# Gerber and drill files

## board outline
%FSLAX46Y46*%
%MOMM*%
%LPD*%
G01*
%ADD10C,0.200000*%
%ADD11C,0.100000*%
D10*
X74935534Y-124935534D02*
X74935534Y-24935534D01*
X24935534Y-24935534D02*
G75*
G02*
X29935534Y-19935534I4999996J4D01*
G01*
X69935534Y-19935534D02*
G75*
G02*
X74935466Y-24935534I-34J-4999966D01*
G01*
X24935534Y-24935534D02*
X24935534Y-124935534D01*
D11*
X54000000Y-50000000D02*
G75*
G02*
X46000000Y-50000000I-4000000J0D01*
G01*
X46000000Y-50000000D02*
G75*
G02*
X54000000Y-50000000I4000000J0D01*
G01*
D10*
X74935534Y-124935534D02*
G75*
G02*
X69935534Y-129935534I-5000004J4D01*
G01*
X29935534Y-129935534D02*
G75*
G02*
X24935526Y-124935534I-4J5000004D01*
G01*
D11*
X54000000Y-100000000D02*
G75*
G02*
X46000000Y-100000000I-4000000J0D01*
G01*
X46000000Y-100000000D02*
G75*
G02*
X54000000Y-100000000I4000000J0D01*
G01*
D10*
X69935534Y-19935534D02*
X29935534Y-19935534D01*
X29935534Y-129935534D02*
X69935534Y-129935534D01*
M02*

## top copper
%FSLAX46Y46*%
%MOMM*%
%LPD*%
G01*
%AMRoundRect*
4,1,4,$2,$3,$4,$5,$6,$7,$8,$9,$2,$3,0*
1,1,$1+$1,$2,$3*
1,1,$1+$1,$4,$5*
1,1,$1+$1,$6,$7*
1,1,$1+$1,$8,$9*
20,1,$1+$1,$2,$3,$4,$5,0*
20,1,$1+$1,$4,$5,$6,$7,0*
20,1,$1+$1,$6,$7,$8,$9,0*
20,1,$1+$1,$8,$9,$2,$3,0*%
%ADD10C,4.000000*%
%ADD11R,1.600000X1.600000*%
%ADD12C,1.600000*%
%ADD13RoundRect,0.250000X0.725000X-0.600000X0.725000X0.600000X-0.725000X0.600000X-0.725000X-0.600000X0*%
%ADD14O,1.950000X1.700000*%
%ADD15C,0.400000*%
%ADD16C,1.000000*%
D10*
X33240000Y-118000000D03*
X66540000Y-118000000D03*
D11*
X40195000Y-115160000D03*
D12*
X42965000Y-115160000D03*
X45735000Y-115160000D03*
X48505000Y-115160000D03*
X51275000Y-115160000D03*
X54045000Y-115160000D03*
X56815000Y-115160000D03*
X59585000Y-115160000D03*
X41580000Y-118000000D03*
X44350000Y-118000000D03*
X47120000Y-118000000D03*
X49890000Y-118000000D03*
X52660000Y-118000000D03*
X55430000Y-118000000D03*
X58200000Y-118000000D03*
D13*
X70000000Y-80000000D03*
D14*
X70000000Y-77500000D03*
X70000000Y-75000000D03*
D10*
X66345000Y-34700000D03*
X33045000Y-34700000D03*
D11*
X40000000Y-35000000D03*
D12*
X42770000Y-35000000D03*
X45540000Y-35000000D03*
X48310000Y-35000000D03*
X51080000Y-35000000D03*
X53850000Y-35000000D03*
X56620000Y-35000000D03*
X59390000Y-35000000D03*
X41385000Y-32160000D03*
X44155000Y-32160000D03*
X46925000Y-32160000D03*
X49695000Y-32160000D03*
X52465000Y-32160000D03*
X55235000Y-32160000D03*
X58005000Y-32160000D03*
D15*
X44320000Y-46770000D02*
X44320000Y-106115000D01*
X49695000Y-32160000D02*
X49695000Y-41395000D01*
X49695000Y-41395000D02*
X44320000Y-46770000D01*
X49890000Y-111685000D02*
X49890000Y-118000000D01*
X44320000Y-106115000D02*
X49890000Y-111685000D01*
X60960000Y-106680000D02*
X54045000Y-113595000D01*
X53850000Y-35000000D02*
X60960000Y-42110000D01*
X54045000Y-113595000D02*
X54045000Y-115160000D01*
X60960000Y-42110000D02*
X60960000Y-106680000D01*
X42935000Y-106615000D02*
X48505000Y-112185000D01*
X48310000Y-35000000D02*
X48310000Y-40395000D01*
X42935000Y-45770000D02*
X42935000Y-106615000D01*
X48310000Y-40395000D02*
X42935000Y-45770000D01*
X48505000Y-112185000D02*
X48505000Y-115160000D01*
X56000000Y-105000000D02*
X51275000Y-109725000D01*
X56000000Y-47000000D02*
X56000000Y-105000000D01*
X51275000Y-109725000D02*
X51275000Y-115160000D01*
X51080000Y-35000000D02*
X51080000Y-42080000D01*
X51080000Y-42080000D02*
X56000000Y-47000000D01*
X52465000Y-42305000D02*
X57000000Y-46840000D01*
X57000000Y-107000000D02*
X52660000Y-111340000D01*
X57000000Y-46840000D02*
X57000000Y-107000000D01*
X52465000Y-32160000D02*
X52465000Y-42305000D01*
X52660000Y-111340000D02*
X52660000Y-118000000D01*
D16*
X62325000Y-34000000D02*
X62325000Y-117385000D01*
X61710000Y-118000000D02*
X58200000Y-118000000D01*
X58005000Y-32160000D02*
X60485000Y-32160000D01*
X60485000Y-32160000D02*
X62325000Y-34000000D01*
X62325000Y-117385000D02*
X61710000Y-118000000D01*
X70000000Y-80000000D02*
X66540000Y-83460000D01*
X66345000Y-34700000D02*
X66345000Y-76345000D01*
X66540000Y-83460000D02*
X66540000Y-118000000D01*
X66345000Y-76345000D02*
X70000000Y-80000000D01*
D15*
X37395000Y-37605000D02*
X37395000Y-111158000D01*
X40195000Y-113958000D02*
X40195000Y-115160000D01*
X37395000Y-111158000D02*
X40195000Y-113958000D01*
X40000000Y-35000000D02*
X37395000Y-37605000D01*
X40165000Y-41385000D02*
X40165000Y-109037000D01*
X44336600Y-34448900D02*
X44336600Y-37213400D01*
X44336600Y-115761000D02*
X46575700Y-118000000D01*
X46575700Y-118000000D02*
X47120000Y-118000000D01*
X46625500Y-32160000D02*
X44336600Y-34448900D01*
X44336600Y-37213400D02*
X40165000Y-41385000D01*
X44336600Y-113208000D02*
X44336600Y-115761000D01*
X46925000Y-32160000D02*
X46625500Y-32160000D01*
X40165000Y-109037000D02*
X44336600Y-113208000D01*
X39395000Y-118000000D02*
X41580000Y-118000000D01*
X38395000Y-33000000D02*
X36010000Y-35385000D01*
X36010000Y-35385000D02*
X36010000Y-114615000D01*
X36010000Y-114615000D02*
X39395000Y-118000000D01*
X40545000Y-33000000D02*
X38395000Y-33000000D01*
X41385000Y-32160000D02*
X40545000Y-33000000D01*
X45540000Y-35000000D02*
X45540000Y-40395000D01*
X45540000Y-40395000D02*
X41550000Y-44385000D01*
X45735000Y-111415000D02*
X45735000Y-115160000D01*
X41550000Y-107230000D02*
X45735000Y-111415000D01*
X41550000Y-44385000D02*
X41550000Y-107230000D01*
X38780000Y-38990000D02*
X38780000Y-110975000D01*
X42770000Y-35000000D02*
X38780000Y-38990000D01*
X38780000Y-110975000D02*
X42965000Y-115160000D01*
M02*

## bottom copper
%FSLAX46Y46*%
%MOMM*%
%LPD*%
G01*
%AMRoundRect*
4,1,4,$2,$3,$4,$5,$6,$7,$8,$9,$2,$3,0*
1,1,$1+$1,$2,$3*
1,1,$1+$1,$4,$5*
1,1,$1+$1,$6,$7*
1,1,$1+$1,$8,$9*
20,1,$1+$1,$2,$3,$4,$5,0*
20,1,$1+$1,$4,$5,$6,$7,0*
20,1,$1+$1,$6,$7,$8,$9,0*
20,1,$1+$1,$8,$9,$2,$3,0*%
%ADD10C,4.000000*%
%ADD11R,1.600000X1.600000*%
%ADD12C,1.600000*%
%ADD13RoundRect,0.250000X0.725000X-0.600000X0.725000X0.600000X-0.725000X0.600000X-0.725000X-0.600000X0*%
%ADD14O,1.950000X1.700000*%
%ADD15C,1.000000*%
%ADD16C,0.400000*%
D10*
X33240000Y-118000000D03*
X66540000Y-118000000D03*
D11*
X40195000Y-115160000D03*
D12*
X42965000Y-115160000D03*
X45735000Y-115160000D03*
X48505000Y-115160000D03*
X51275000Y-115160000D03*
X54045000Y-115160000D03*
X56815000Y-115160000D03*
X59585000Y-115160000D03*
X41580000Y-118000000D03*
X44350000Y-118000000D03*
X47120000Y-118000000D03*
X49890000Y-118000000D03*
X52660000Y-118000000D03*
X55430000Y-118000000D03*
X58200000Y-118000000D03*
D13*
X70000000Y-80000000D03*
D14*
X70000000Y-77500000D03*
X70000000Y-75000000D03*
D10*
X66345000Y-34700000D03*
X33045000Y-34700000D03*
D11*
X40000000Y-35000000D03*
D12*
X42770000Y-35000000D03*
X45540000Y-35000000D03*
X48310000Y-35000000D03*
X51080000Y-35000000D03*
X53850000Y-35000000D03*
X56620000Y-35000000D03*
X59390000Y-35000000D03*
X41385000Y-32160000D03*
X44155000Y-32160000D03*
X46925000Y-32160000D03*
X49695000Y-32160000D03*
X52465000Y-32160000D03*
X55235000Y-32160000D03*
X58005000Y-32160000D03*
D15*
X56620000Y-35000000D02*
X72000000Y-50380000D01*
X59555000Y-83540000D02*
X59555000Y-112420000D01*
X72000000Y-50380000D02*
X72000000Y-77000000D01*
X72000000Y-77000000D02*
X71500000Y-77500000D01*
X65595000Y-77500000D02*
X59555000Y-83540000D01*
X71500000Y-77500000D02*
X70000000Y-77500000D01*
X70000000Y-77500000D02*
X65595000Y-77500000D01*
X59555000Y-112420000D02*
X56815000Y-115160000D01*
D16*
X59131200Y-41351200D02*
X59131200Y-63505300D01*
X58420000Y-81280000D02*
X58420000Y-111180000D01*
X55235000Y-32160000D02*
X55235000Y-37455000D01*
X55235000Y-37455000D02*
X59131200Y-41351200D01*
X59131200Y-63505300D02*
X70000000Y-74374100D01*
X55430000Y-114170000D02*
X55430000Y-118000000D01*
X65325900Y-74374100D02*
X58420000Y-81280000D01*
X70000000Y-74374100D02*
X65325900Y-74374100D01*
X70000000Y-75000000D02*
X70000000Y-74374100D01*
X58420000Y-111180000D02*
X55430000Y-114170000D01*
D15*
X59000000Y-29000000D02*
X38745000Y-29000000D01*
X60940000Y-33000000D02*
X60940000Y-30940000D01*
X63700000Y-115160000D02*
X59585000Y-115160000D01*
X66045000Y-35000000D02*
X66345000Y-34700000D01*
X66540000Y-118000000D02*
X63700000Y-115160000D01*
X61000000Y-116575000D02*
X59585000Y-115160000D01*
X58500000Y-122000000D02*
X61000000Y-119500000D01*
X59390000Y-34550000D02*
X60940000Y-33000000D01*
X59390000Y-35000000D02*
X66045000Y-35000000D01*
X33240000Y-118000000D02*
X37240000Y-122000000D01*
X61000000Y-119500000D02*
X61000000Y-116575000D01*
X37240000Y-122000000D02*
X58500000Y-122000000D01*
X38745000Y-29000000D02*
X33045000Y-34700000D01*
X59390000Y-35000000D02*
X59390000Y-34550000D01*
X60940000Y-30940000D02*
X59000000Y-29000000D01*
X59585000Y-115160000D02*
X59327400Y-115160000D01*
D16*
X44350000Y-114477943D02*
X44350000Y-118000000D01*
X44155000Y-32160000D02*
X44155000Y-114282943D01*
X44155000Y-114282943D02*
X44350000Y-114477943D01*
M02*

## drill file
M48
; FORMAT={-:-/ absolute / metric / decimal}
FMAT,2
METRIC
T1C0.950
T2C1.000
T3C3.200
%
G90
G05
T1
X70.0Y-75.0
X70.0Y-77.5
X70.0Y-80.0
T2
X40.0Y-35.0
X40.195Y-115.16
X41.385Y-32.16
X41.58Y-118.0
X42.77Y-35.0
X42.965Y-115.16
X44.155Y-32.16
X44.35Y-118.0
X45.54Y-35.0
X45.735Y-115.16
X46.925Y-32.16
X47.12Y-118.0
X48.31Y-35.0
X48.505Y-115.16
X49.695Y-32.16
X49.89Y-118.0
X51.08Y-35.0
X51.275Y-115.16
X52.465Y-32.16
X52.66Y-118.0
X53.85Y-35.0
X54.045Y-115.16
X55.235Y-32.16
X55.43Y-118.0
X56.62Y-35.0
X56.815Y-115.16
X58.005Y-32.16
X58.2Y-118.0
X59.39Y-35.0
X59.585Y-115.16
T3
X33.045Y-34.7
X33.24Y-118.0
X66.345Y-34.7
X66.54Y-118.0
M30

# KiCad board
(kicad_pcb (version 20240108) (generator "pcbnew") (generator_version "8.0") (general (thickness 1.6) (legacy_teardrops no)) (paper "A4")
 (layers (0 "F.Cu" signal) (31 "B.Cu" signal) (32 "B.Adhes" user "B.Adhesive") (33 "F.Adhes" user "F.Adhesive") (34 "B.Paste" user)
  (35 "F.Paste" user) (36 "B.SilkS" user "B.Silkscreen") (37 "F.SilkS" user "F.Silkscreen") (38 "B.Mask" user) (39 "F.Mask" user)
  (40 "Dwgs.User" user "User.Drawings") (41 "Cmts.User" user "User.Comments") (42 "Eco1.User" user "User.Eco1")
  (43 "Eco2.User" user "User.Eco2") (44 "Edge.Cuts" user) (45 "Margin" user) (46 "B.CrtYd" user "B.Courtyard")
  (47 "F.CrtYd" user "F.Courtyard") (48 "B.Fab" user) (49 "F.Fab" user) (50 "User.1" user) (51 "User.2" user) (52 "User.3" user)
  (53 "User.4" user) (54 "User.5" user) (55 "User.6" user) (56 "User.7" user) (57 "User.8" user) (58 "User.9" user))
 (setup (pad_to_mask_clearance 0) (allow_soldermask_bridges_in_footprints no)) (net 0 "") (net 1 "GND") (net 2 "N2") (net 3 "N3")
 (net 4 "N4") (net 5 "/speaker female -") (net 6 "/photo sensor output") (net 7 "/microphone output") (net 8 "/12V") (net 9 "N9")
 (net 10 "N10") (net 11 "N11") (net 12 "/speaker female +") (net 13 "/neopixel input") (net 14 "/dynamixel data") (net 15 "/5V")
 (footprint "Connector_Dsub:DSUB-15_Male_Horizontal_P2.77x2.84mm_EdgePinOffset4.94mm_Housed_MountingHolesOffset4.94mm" (layer "F.Cu")
  (at 40.195 115.16)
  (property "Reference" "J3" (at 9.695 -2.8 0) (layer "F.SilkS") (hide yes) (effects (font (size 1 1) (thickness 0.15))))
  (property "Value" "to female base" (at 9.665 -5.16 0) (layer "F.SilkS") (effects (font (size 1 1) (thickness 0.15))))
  (pad "0" thru_hole circle (at -6.955 2.84) (size 4 4) (drill 3.2) (layers "*.Cu" "*.Mask") (remove_unused_layers no) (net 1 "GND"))
  (pad "0" thru_hole circle (at 26.345 2.84) (size 4 4) (drill 3.2) (layers "*.Cu" "*.Mask") (remove_unused_layers no) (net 1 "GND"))
  (pad "1" thru_hole rect (at 0 0) (size 1.6 1.6) (drill 1) (layers "*.Cu" "*.Mask") (remove_unused_layers no) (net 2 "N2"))
  (pad "2" thru_hole circle (at 2.77 0) (size 1.6 1.6) (drill 1) (layers "*.Cu" "*.Mask") (remove_unused_layers no) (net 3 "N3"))
  (pad "3" thru_hole circle (at 5.54 0) (size 1.6 1.6) (drill 1) (layers "*.Cu" "*.Mask") (remove_unused_layers no) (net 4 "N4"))
  (pad "4" thru_hole circle (at 8.31 0) (size 1.6 1.6) (drill 1) (layers "*.Cu" "*.Mask") (remove_unused_layers no)
   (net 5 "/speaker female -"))
  (pad "5" thru_hole circle (at 11.08 0) (size 1.6 1.6) (drill 1) (layers "*.Cu" "*.Mask") (remove_unused_layers no)
   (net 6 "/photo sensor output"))
  (pad "6" thru_hole circle (at 13.85 0) (size 1.6 1.6) (drill 1) (layers "*.Cu" "*.Mask") (remove_unused_layers no)
   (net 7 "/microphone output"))
  (pad "7" thru_hole circle (at 16.62 0) (size 1.6 1.6) (drill 1) (layers "*.Cu" "*.Mask") (remove_unused_layers no) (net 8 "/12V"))
  (pad "8" thru_hole circle (at 19.39 0) (size 1.6 1.6) (drill 1) (layers "*.Cu" "*.Mask") (remove_unused_layers no) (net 1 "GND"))
  (pad "9" thru_hole circle (at 1.385 2.84) (size 1.6 1.6) (drill 1) (layers "*.Cu" "*.Mask") (remove_unused_layers no) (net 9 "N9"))
  (pad "10" thru_hole circle (at 4.155 2.84) (size 1.6 1.6) (drill 1) (layers "*.Cu" "*.Mask") (remove_unused_layers no) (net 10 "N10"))
  (pad "11" thru_hole circle (at 6.925 2.84) (size 1.6 1.6) (drill 1) (layers "*.Cu" "*.Mask") (remove_unused_layers no) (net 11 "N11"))
  (pad "12" thru_hole circle (at 9.695 2.84) (size 1.6 1.6) (drill 1) (layers "*.Cu" "*.Mask") (remove_unused_layers no)
   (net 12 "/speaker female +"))
  (pad "13" thru_hole circle (at 12.465 2.84) (size 1.6 1.6) (drill 1) (layers "*.Cu" "*.Mask") (remove_unused_layers no)
   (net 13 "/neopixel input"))
  (pad "14" thru_hole circle (at 15.235 2.84) (size 1.6 1.6) (drill 1) (layers "*.Cu" "*.Mask") (remove_unused_layers no)
   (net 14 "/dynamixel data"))
  (pad "15" thru_hole circle (at 18.005 2.84) (size 1.6 1.6) (drill 1) (layers "*.Cu" "*.Mask") (remove_unused_layers no) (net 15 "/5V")))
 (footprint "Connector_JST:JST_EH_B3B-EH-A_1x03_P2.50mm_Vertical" (layer "F.Cu") (at 70 80 90)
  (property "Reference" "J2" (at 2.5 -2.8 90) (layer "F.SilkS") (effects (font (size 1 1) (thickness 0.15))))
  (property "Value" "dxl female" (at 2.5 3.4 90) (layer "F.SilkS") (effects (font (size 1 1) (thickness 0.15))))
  (pad "1" thru_hole roundrect (at 0 0 90) (size 1.7 1.95) (drill 0.95) (layers "*.Cu" "*.Mask") (remove_unused_layers no)
   (roundrect_rratio 0.147059) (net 1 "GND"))
  (pad "2" thru_hole oval (at 2.5 0 90) (size 1.7 1.95) (drill 0.95) (layers "*.Cu" "*.Mask") (remove_unused_layers no) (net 8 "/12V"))
  (pad "3" thru_hole oval (at 5 0 90) (size 1.7 1.95) (drill 0.95) (layers "*.Cu" "*.Mask") (remove_unused_layers no)
   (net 14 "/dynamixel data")))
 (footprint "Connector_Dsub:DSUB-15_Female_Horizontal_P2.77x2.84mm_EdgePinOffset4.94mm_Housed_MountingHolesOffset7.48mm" (layer "F.Cu")
  (at 40 35 180)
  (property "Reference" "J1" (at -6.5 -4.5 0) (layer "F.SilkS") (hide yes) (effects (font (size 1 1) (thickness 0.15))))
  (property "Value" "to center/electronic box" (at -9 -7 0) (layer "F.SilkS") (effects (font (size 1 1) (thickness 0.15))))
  (pad "0" thru_hole circle (at -26.345 0.3 180) (size 4 4) (drill 3.2) (layers "*.Cu" "*.Mask") (remove_unused_layers no) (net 1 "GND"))
  (pad "0" thru_hole circle (at 6.955 0.3 180) (size 4 4) (drill 3.2) (layers "*.Cu" "*.Mask") (remove_unused_layers no) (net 1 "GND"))
  (pad "1" thru_hole rect (at 0 0 180) (size 1.6 1.6) (drill 1) (layers "*.Cu" "*.Mask") (remove_unused_layers no) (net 2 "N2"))
  (pad "2" thru_hole circle (at -2.77 0 180) (size 1.6 1.6) (drill 1) (layers "*.Cu" "*.Mask") (remove_unused_layers no) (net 3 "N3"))
  (pad "3" thru_hole circle (at -5.54 0 180) (size 1.6 1.6) (drill 1) (layers "*.Cu" "*.Mask") (remove_unused_layers no) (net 4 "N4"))
  (pad "4" thru_hole circle (at -8.31 0 180) (size 1.6 1.6) (drill 1) (layers "*.Cu" "*.Mask") (remove_unused_layers no)
   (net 5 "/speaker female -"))
  (pad "5" thru_hole circle (at -11.08 0 180) (size 1.6 1.6) (drill 1) (layers "*.Cu" "*.Mask") (remove_unused_layers no)
   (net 6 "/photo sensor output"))
  (pad "6" thru_hole circle (at -13.85 0 180) (size 1.6 1.6) (drill 1) (layers "*.Cu" "*.Mask") (remove_unused_layers no)
   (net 7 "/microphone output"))
  (pad "7" thru_hole circle (at -16.62 0 180) (size 1.6 1.6) (drill 1) (layers "*.Cu" "*.Mask") (remove_unused_layers no) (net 8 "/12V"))
  (pad "8" thru_hole circle (at -19.39 0 180) (size 1.6 1.6) (drill 1) (layers "*.Cu" "*.Mask") (remove_unused_layers no) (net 1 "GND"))
  (pad "9" thru_hole circle (at -1.385 2.84 180) (size 1.6 1.6) (drill 1) (layers "*.Cu" "*.Mask") (remove_unused_layers no) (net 9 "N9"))
  (pad "10" thru_hole circle (at -4.155 2.84 180) (size 1.6 1.6) (drill 1) (layers "*.Cu" "*.Mask") (remove_unused_layers no) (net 10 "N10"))
  (pad "11" thru_hole circle (at -6.925 2.84 180) (size 1.6 1.6) (drill 1) (layers "*.Cu" "*.Mask") (remove_unused_layers no) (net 11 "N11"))
  (pad "12" thru_hole circle (at -9.695 2.84 180) (size 1.6 1.6) (drill 1) (layers "*.Cu" "*.Mask") (remove_unused_layers no)
   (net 12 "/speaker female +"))
  (pad "13" thru_hole circle (at -12.465 2.84 180) (size 1.6 1.6) (drill 1) (layers "*.Cu" "*.Mask") (remove_unused_layers no)
   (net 13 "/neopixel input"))
  (pad "14" thru_hole circle (at -15.235 2.84 180) (size 1.6 1.6) (drill 1) (layers "*.Cu" "*.Mask") (remove_unused_layers no)
   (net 14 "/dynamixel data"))
  (pad "15" thru_hole circle (at -18.005 2.84 180) (size 1.6 1.6) (drill 1) (layers "*.Cu" "*.Mask") (remove_unused_layers no)
   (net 15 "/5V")))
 (gr_line (start 74.935534 124.935534) (end 74.935534 24.935534) (stroke (width 0.2) (type default)) (layer "Edge.Cuts"))
 (gr_arc (start 24.935534 24.935534) (mid 26.4 21.4) (end 29.935534 19.935534) (stroke (width 0.2) (type default)) (layer "Edge.Cuts"))
 (gr_arc (start 69.935534 19.935534) (mid 73.471068 21.4) (end 74.935534 24.935534) (stroke (width 0.2) (type default)) (layer "Edge.Cuts"))
 (gr_line (start 24.935534 24.935534) (end 24.935534 124.935534) (stroke (width 0.2) (type default)) (layer "Edge.Cuts"))
 (gr_circle (center 50 50) (end 54 50) (stroke (width 0.1) (type default)) (fill none) (layer "Edge.Cuts"))
 (gr_arc (start 74.935534 124.935534) (mid 73.471068 128.471068) (end 69.935534 129.935534) (stroke (width 0.2) (type default))
  (layer "Edge.Cuts"))
 (gr_arc (start 29.935534 129.935534) (mid 26.4 128.471068) (end 24.935534 124.935534) (stroke (width 0.2) (type default))
  (layer "Edge.Cuts"))
 (gr_circle (center 50 100) (end 54 100) (stroke (width 0.1) (type default)) (fill none) (layer "Edge.Cuts"))
 (gr_line (start 69.935534 19.935534) (end 29.935534 19.935534) (stroke (width 0.2) (type default)) (layer "Edge.Cuts"))
 (gr_line (start 29.935534 129.935534) (end 69.935534 129.935534) (stroke (width 0.2) (type default)) (layer "Edge.Cuts"))
 (segment (start 44.32 46.77) (end 44.32 106.115) (width 0.4) (layer "F.Cu") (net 12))
 (segment (start 49.695 32.16) (end 49.695 41.395) (width 0.4) (layer "F.Cu") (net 12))
 (segment (start 49.695 41.395) (end 44.32 46.77) (width 0.4) (layer "F.Cu") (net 12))
 (segment (start 49.89 111.685) (end 49.89 118) (width 0.4) (layer "F.Cu") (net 12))
 (segment (start 44.32 106.115) (end 49.89 111.685) (width 0.4) (layer "F.Cu") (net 12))
 (segment (start 56.62 35) (end 72 50.38) (width 1) (layer "B.Cu") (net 8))
 (segment (start 59.555 83.54) (end 59.555 112.42) (width 1) (layer "B.Cu") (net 8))
 (segment (start 72 50.38) (end 72 77) (width 1) (layer "B.Cu") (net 8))
 (segment (start 72 77) (end 71.5 77.5) (width 1) (layer "B.Cu") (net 8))
 (segment (start 65.595 77.5) (end 59.555 83.54) (width 1) (layer "B.Cu") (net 8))
 (segment (start 71.5 77.5) (end 70 77.5) (width 1) (layer "B.Cu") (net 8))
 (segment (start 70 77.5) (end 65.595 77.5) (width 1) (layer "B.Cu") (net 8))
 (segment (start 59.555 112.42) (end 56.815 115.16) (width 1) (layer "B.Cu") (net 8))
 (segment (start 59.1312 41.3512) (end 59.1312 63.5053) (width 0.4) (layer "B.Cu") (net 14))
 (segment (start 58.42 81.28) (end 58.42 111.18) (width 0.4) (layer "B.Cu") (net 14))
 (segment (start 55.235 32.16) (end 55.235 37.455) (width 0.4) (layer "B.Cu") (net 14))
 (segment (start 55.235 37.455) (end 59.1312 41.3512) (width 0.4) (layer "B.Cu") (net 14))
 (segment (start 59.1312 63.5053) (end 70 74.3741) (width 0.4) (layer "B.Cu") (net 14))
 (segment (start 55.43 114.17) (end 55.43 118) (width 0.4) (layer "B.Cu") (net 14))
 (segment (start 65.3259 74.3741) (end 58.42 81.28) (width 0.4) (layer "B.Cu") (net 14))
 (segment (start 70 74.3741) (end 65.3259 74.3741) (width 0.4) (layer "B.Cu") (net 14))
 (segment (start 70 75) (end 70 74.3741) (width 0.4) (layer "B.Cu") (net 14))
 (segment (start 58.42 111.18) (end 55.43 114.17) (width 0.4) (layer "B.Cu") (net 14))
 (segment (start 60.96 106.68) (end 54.045 113.595) (width 0.4) (layer "F.Cu") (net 7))
 (segment (start 53.85 35) (end 60.96 42.11) (width 0.4) (layer "F.Cu") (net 7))
 (segment (start 54.045 113.595) (end 54.045 115.16) (width 0.4) (layer "F.Cu") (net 7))
 (segment (start 60.96 42.11) (end 60.96 106.68) (width 0.4) (layer "F.Cu") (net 7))
 (segment (start 42.935 106.615) (end 48.505 112.185) (width 0.4) (layer "F.Cu") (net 5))
 (segment (start 48.31 35) (end 48.31 40.395) (width 0.4) (layer "F.Cu") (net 5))
 (segment (start 42.935 45.77) (end 42.935 106.615) (width 0.4) (layer "F.Cu") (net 5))
 (segment (start 48.31 40.395) (end 42.935 45.77) (width 0.4) (layer "F.Cu") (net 5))
 (segment (start 48.505 112.185) (end 48.505 115.16) (width 0.4) (layer "F.Cu") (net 5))
 (segment (start 56 105) (end 51.275 109.725) (width 0.4) (layer "F.Cu") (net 6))
 (segment (start 56 47) (end 56 105) (width 0.4) (layer "F.Cu") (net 6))
 (segment (start 51.275 109.725) (end 51.275 115.16) (width 0.4) (layer "F.Cu") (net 6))
 (segment (start 51.08 35) (end 51.08 42.08) (width 0.4) (layer "F.Cu") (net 6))
 (segment (start 51.08 42.08) (end 56 47) (width 0.4) (layer "F.Cu") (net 6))
 (segment (start 52.465 42.305) (end 57 46.84) (width 0.4) (layer "F.Cu") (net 13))
 (segment (start 57 107) (end 52.66 111.34) (width 0.4) (layer "F.Cu") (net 13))
 (segment (start 57 46.84) (end 57 107) (width 0.4) (layer "F.Cu") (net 13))
 (segment (start 52.465 32.16) (end 52.465 42.305) (width 0.4) (layer "F.Cu") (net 13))
 (segment (start 52.66 111.34) (end 52.66 118) (width 0.4) (layer "F.Cu") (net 13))
 (segment (start 62.325 34) (end 62.325 117.385) (width 1) (layer "F.Cu") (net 15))
 (segment (start 61.71 118) (end 58.2 118) (width 1) (layer "F.Cu") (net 15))
 (segment (start 58.005 32.16) (end 60.485 32.16) (width 1) (layer "F.Cu") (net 15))
 (segment (start 60.485 32.16) (end 62.325 34) (width 1) (layer "F.Cu") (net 15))
 (segment (start 62.325 117.385) (end 61.71 118) (width 1) (layer "F.Cu") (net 15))
 (segment (start 70 80) (end 66.54 83.46) (width 1) (layer "F.Cu") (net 1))
 (segment (start 66.345 34.7) (end 66.345 76.345) (width 1) (layer "F.Cu") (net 1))
 (segment (start 66.54 83.46) (end 66.54 118) (width 1) (layer "F.Cu") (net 1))
 (segment (start 66.345 76.345) (end 70 80) (width 1) (layer "F.Cu") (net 1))
 (segment (start 59 29) (end 38.745 29) (width 1) (layer "B.Cu") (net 1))
 (segment (start 60.94 33) (end 60.94 30.94) (width 1) (layer "B.Cu") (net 1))
 (segment (start 63.7 115.16) (end 59.585 115.16) (width 1) (layer "B.Cu") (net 1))
 (segment (start 66.045 35) (end 66.345 34.7) (width 1) (layer "B.Cu") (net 1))
 (segment (start 66.54 118) (end 63.7 115.16) (width 1) (layer "B.Cu") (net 1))
 (segment (start 61 116.575) (end 59.585 115.16) (width 1) (layer "B.Cu") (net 1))
 (segment (start 58.5 122) (end 61 119.5) (width 1) (layer "B.Cu") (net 1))
 (segment (start 59.39 34.55) (end 60.94 33) (width 1) (layer "B.Cu") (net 1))
 (segment (start 59.39 35) (end 66.045 35) (width 1) (layer "B.Cu") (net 1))
 (segment (start 33.24 118) (end 37.24 122) (width 1) (layer "B.Cu") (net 1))
 (segment (start 61 119.5) (end 61 116.575) (width 1) (layer "B.Cu") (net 1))
 (segment (start 37.24 122) (end 58.5 122) (width 1) (layer "B.Cu") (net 1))
 (segment (start 38.745 29) (end 33.045 34.7) (width 1) (layer "B.Cu") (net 1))
 (segment (start 59.39 35) (end 59.39 34.55) (width 1) (layer "B.Cu") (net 1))
 (segment (start 60.94 30.94) (end 59 29) (width 1) (layer "B.Cu") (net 1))
 (segment (start 59.585 115.16) (end 59.3274 115.16) (width 1) (layer "B.Cu") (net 1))
 (segment (start 37.395 37.605) (end 37.395 111.158) (width 0.4) (layer "F.Cu") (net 2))
 (segment (start 40.195 113.958) (end 40.195 115.16) (width 0.4) (layer "F.Cu") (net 2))
 (segment (start 37.395 111.158) (end 40.195 113.958) (width 0.4) (layer "F.Cu") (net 2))
 (segment (start 40 35) (end 37.395 37.605) (width 0.4) (layer "F.Cu") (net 2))
 (segment (start 40.165 41.385) (end 40.165 109.037) (width 0.4) (layer "F.Cu") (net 11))
 (segment (start 44.3366 34.4489) (end 44.3366 37.2134) (width 0.4) (layer "F.Cu") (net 11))
 (segment (start 44.3366 115.761) (end 46.5757 118) (width 0.4) (layer "F.Cu") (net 11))
 (segment (start 46.5757 118) (end 47.12 118) (width 0.4) (layer "F.Cu") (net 11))
 (segment (start 46.6255 32.16) (end 44.3366 34.4489) (width 0.4) (layer "F.Cu") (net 11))
 (segment (start 44.3366 37.2134) (end 40.165 41.385) (width 0.4) (layer "F.Cu") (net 11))
 (segment (start 44.3366 113.208) (end 44.3366 115.761) (width 0.4) (layer "F.Cu") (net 11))
 (segment (start 46.925 32.16) (end 46.6255 32.16) (width 0.4) (layer "F.Cu") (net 11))
 (segment (start 40.165 109.037) (end 44.3366 113.208) (width 0.4) (layer "F.Cu") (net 11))
 (segment (start 39.395 118) (end 41.58 118) (width 0.4) (layer "F.Cu") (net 9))
 (segment (start 38.395 33) (end 36.01 35.385) (width 0.4) (layer "F.Cu") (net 9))
 (segment (start 36.01 35.385) (end 36.01 114.615) (width 0.4) (layer "F.Cu") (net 9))
 (segment (start 36.01 114.615) (end 39.395 118) (width 0.4) (layer "F.Cu") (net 9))
 (segment (start 40.545 33) (end 38.395 33) (width 0.4) (layer "F.Cu") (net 9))
 (segment (start 41.385 32.16) (end 40.545 33) (width 0.4) (layer "F.Cu") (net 9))
 (segment (start 45.54 35) (end 45.54 40.395) (width 0.4) (layer "F.Cu") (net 4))
 (segment (start 45.54 40.395) (end 41.55 44.385) (width 0.4) (layer "F.Cu") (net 4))
 (segment (start 45.735 111.415) (end 45.735 115.16) (width 0.4) (layer "F.Cu") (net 4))
 (segment (start 41.55 107.23) (end 45.735 111.415) (width 0.4) (layer "F.Cu") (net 4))
 (segment (start 41.55 44.385) (end 41.55 107.23) (width 0.4) (layer "F.Cu") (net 4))
 (segment (start 44.35 114.477943) (end 44.35 118) (width 0.4) (layer "B.Cu") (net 10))
 (segment (start 44.155 32.16) (end 44.155 114.282943) (width 0.4) (layer "B.Cu") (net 10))
 (segment (start 44.155 114.282943) (end 44.35 114.477943) (width 0.4) (layer "B.Cu") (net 10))
 (segment (start 38.78 38.99) (end 38.78 110.975) (width 0.4) (layer "F.Cu") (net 3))
 (segment (start 42.77 35) (end 38.78 38.99) (width 0.4) (layer "F.Cu") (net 3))
 (segment (start 38.78 110.975) (end 42.965 115.16) (width 0.4) (layer "F.Cu") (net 3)))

